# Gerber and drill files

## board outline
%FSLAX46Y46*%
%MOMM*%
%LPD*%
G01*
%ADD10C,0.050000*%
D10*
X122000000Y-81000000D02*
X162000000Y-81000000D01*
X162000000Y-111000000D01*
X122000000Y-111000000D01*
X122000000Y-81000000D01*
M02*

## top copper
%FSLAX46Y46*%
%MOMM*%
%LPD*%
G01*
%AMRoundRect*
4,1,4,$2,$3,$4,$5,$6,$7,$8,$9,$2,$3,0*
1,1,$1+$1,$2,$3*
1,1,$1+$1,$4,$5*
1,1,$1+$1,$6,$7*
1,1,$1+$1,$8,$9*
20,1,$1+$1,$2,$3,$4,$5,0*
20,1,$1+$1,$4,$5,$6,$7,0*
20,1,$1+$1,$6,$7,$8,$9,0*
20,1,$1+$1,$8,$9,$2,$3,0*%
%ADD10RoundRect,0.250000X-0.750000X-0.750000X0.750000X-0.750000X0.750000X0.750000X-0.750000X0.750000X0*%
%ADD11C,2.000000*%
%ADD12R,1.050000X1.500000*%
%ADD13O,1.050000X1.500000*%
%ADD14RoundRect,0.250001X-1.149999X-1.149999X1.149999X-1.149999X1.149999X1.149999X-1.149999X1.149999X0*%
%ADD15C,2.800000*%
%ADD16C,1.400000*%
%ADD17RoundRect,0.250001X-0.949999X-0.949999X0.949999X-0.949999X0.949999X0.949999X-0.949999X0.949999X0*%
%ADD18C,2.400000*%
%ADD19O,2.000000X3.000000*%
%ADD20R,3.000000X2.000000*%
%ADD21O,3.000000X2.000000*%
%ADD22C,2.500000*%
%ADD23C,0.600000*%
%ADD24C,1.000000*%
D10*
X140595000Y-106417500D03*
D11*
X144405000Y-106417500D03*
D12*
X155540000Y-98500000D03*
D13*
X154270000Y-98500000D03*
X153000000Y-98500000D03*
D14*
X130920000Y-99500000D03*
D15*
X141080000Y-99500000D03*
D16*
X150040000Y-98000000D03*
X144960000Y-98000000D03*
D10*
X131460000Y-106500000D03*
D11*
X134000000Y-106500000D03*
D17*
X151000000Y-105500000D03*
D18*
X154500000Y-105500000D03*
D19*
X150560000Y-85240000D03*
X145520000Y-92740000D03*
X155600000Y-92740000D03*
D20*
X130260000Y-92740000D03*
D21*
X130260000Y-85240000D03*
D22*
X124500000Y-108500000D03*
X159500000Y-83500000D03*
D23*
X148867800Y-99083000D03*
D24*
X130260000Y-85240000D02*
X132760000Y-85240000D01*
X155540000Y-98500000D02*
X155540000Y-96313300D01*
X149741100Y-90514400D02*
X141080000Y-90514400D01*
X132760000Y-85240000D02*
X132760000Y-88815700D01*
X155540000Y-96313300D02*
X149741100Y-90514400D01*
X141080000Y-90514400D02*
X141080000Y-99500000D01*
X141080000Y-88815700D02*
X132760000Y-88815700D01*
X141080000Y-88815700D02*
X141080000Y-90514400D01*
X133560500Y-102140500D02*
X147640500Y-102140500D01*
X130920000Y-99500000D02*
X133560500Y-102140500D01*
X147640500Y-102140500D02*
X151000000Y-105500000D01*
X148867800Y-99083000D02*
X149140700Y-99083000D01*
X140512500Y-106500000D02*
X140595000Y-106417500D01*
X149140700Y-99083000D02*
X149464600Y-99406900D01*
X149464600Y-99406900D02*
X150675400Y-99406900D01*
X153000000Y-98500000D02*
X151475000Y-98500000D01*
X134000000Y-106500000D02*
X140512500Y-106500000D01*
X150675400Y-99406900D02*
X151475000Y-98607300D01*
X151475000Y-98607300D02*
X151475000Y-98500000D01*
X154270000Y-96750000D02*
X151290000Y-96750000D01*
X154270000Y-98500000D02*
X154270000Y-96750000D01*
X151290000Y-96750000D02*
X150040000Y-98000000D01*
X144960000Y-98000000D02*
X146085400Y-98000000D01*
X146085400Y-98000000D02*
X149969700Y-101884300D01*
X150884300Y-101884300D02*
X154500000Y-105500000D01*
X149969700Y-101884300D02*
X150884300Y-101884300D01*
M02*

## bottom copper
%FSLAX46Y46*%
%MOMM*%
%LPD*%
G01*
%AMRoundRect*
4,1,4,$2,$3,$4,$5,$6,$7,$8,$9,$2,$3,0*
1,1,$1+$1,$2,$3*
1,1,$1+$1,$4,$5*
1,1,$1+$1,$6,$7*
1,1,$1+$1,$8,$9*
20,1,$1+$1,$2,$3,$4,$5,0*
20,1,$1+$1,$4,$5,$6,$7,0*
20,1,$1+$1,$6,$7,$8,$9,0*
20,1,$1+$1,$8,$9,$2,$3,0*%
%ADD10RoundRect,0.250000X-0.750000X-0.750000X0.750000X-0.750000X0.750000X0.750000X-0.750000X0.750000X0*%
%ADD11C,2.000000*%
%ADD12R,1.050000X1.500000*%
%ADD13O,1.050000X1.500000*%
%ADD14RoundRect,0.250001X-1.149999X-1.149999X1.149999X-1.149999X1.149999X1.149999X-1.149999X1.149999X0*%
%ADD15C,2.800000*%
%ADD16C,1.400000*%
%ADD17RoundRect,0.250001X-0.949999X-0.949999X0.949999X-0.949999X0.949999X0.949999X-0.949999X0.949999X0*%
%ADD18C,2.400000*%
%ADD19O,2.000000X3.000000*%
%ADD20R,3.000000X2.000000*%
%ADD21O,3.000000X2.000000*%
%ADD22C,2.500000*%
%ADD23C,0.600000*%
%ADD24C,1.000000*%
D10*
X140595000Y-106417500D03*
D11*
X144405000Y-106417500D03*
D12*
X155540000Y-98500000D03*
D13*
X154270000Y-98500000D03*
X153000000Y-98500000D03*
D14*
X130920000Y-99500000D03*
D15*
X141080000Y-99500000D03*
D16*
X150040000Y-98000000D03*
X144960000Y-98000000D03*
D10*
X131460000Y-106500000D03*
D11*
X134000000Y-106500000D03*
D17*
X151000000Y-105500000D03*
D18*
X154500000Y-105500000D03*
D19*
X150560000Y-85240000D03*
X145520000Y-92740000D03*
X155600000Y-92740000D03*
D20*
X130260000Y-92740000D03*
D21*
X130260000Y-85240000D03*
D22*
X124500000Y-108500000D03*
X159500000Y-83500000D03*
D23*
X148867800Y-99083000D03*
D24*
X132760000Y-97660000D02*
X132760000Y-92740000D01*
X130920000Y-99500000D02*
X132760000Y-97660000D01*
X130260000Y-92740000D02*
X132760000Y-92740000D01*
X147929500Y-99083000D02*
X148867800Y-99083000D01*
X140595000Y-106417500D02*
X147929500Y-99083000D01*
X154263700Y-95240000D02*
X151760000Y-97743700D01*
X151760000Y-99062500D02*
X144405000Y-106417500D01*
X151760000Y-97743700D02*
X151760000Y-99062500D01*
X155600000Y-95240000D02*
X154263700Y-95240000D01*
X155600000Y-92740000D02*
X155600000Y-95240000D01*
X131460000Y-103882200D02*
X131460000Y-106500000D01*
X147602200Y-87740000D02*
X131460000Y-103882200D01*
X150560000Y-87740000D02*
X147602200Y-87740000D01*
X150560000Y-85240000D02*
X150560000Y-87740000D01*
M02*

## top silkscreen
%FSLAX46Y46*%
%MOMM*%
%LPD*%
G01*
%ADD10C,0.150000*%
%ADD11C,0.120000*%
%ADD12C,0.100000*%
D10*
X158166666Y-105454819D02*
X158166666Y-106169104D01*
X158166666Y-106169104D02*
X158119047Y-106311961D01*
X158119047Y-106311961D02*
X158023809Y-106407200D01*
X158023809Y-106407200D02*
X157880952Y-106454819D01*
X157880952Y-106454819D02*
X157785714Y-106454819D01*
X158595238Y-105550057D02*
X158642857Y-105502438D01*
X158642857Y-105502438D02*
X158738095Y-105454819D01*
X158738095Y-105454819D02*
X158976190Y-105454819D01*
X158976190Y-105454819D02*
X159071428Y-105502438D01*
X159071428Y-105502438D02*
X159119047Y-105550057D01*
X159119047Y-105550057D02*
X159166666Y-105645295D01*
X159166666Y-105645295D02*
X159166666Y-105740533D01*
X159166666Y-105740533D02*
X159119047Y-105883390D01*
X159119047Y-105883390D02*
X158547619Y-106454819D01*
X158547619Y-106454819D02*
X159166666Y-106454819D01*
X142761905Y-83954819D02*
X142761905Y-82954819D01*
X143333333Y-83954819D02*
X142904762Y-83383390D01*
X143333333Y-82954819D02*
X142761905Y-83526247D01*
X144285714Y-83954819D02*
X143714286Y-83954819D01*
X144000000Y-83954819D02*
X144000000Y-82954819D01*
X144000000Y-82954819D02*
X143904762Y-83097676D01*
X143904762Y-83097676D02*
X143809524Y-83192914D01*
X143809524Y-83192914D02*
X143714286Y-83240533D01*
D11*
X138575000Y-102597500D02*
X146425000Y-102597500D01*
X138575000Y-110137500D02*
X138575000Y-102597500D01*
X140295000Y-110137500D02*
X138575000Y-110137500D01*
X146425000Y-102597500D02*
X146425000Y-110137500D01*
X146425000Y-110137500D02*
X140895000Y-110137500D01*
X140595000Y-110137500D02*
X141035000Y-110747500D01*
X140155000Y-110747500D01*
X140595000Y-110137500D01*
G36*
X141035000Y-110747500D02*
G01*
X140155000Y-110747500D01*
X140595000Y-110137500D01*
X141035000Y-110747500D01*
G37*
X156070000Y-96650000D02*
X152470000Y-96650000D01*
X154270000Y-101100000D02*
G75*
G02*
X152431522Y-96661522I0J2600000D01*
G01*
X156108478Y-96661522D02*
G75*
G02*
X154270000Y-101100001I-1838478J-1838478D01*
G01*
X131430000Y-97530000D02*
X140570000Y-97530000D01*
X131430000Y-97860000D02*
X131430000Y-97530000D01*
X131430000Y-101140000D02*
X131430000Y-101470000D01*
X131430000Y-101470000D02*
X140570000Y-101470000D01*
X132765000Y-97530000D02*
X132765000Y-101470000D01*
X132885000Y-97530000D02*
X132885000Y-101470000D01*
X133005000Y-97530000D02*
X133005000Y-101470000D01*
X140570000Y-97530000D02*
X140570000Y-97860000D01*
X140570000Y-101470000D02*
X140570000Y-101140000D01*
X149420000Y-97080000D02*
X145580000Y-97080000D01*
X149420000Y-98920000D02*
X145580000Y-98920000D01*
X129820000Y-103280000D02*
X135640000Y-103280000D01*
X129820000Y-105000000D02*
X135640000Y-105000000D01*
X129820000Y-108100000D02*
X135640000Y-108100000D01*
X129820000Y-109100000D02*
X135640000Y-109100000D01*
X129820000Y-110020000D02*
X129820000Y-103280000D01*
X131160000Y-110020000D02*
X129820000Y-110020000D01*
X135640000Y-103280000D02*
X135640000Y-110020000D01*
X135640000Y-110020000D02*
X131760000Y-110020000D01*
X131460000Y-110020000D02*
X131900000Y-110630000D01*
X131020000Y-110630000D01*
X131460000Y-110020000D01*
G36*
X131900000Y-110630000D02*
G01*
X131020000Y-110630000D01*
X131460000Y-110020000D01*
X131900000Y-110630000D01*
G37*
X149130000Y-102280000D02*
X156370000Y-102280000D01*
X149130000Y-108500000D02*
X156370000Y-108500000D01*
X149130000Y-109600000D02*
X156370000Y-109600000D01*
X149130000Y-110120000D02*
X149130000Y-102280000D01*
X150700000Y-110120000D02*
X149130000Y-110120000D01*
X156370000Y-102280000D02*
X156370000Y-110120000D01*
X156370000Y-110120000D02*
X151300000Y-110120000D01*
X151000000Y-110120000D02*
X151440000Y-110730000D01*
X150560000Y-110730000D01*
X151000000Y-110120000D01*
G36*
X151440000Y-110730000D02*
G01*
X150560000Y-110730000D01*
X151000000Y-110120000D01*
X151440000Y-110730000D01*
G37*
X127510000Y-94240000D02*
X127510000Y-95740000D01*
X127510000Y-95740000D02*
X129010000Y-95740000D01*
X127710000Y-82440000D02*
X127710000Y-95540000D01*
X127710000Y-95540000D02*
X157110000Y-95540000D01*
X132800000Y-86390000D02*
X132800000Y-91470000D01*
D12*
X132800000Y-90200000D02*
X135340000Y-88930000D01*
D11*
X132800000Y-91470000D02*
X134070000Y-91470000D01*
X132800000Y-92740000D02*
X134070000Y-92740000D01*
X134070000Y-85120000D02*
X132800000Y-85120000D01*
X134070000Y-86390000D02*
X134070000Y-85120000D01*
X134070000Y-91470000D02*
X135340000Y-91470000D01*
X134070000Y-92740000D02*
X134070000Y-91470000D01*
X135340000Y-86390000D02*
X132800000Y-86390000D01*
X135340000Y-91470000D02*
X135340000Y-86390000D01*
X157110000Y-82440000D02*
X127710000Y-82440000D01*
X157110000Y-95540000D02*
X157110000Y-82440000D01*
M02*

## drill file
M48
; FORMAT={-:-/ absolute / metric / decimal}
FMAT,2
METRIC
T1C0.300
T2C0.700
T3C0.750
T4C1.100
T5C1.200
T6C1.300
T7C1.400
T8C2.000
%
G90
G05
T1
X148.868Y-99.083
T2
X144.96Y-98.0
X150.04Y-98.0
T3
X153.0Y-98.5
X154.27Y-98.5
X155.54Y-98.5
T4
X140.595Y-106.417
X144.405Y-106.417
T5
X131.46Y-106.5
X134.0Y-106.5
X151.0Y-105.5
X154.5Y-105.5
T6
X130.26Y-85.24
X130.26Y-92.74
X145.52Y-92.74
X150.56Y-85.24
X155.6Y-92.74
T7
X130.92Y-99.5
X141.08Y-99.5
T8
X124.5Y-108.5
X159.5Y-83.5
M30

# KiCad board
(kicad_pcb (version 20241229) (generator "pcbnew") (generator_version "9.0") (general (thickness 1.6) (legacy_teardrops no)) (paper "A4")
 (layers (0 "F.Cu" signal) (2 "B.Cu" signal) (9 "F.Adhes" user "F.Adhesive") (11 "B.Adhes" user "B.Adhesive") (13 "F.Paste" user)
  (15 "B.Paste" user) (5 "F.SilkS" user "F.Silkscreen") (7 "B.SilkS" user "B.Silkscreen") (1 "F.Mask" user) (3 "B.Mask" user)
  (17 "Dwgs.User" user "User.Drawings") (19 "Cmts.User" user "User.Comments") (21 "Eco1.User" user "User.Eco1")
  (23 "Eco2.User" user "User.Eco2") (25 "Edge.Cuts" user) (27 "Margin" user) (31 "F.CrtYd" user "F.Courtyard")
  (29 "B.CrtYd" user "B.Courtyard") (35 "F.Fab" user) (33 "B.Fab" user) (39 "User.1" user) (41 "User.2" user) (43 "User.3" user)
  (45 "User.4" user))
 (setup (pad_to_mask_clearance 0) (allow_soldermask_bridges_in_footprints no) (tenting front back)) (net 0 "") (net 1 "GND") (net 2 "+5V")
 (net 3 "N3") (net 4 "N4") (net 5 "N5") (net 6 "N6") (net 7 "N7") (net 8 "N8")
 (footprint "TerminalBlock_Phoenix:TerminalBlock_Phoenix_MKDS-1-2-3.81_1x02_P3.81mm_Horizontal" (layer "F.Cu") (at 140.595 106.4175)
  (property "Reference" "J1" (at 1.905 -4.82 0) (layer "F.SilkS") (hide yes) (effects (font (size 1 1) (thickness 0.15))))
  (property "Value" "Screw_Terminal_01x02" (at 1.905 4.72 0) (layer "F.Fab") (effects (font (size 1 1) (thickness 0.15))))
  (fp_line (start -2.02 -3.82) (end 5.83 -3.82) (stroke (width 0.12) (type solid)) (layer "F.SilkS"))
  (fp_line (start -2.02 3.72) (end -2.02 -3.82) (stroke (width 0.12) (type solid)) (layer "F.SilkS"))
  (fp_line (start -0.3 3.72) (end -2.02 3.72) (stroke (width 0.12) (type solid)) (layer "F.SilkS"))
  (fp_line (start 5.83 -3.82) (end 5.83 3.72) (stroke (width 0.12) (type solid)) (layer "F.SilkS"))
  (fp_line (start 5.83 3.72) (end 0.3 3.72) (stroke (width 0.12) (type solid)) (layer "F.SilkS"))
  (fp_poly (pts (xy 0 3.72) (xy 0.44 4.33) (xy -0.44 4.33)) (stroke (width 0.12) (type solid)) (fill yes) (layer "F.SilkS"))
  (pad "1" thru_hole roundrect (at 0 0) (size 2 2) (drill 1.1) (layers "*.Cu" "*.Mask") (remove_unused_layers no) (roundrect_rratio 0.125)
   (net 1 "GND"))
  (pad "2" thru_hole circle (at 3.81 0) (size 2 2) (drill 1.1) (layers "*.Cu" "*.Mask") (remove_unused_layers no) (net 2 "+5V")))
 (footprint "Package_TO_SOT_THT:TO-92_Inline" (layer "F.Cu") (at 155.54 98.5 180)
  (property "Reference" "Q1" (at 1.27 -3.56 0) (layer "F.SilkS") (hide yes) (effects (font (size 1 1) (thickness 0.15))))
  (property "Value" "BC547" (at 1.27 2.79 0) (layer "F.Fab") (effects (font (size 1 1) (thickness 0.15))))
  (fp_line (start -0.53 1.85) (end 3.07 1.85) (stroke (width 0.12) (type solid)) (layer "F.SilkS"))
  (fp_arc (start 1.27 -2.6) (mid 3.672087 -0.994977) (end 3.108478 1.838478) (stroke (width 0.12) (type solid)) (layer "F.SilkS"))
  (fp_arc (start -0.568478 1.838478) (mid -1.132087 -0.994977) (end 1.27 -2.6) (stroke (width 0.12) (type solid)) (layer "F.SilkS"))
  (pad "1" thru_hole rect (at 0 0 180) (size 1.05 1.5) (drill 0.75) (layers "*.Cu" "*.Mask") (remove_unused_layers no) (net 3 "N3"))
  (pad "2" thru_hole oval (at 1.27 0 180) (size 1.05 1.5) (drill 0.75) (layers "*.Cu" "*.Mask") (remove_unused_layers no) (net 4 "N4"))
  (pad "3" thru_hole oval (at 2.54 0 180) (size 1.05 1.5) (drill 0.75) (layers "*.Cu" "*.Mask") (remove_unused_layers no) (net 1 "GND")))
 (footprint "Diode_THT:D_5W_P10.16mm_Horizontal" (layer "F.Cu") (at 130.92 99.5)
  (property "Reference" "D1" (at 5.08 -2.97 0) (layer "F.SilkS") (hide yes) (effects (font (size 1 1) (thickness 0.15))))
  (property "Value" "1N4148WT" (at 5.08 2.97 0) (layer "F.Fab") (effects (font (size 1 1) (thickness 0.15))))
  (fp_line (start 0.51 -1.97) (end 9.65 -1.97) (stroke (width 0.12) (type solid)) (layer "F.SilkS"))
  (fp_line (start 0.51 -1.64) (end 0.51 -1.97) (stroke (width 0.12) (type solid)) (layer "F.SilkS"))
  (fp_line (start 0.51 1.64) (end 0.51 1.97) (stroke (width 0.12) (type solid)) (layer "F.SilkS"))
  (fp_line (start 0.51 1.97) (end 9.65 1.97) (stroke (width 0.12) (type solid)) (layer "F.SilkS"))
  (fp_line (start 1.845 -1.97) (end 1.845 1.97) (stroke (width 0.12) (type solid)) (layer "F.SilkS"))
  (fp_line (start 1.965 -1.97) (end 1.965 1.97) (stroke (width 0.12) (type solid)) (layer "F.SilkS"))
  (fp_line (start 2.085 -1.97) (end 2.085 1.97) (stroke (width 0.12) (type solid)) (layer "F.SilkS"))
  (fp_line (start 9.65 -1.97) (end 9.65 -1.64) (stroke (width 0.12) (type solid)) (layer "F.SilkS"))
  (fp_line (start 9.65 1.97) (end 9.65 1.64) (stroke (width 0.12) (type solid)) (layer "F.SilkS"))
  (pad "1" thru_hole roundrect (at 0 0) (size 2.8 2.8) (drill 1.4) (layers "*.Cu" "*.Mask") (remove_unused_layers no)
   (roundrect_rratio 0.089286) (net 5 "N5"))
  (pad "2" thru_hole circle (at 10.16 0) (size 2.8 2.8) (drill 1.4) (layers "*.Cu" "*.Mask") (remove_unused_layers no) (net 3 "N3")))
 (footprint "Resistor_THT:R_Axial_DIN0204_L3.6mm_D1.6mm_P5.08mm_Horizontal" (layer "F.Cu") (at 150.04 98 180)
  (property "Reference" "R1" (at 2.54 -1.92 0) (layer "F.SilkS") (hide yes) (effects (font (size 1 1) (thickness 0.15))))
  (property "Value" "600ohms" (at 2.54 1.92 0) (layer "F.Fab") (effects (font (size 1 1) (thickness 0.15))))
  (fp_line (start 0.62 0.92) (end 4.46 0.92) (stroke (width 0.12) (type solid)) (layer "F.SilkS"))
  (fp_line (start 0.62 -0.92) (end 4.46 -0.92) (stroke (width 0.12) (type solid)) (layer "F.SilkS"))
  (pad "1" thru_hole circle (at 0 0 180) (size 1.4 1.4) (drill 0.7) (layers "*.Cu" "*.Mask") (remove_unused_layers no) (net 4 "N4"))
  (pad "2" thru_hole circle (at 5.08 0 180) (size 1.4 1.4) (drill 0.7) (layers "*.Cu" "*.Mask") (remove_unused_layers no) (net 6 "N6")))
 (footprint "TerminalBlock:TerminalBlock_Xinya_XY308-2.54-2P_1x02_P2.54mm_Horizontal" (layer "F.Cu") (at 131.46 106.5)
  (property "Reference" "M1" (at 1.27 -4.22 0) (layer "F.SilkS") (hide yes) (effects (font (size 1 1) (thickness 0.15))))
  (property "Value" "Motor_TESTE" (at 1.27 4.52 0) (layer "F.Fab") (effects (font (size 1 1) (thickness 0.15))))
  (fp_line (start -1.64 -3.22) (end 4.18 -3.22) (stroke (width 0.12) (type solid)) (layer "F.SilkS"))
  (fp_line (start -1.64 -1.5) (end 4.18 -1.5) (stroke (width 0.12) (type solid)) (layer "F.SilkS"))
  (fp_line (start -1.64 1.6) (end 4.18 1.6) (stroke (width 0.12) (type solid)) (layer "F.SilkS"))
  (fp_line (start -1.64 2.6) (end 4.18 2.6) (stroke (width 0.12) (type solid)) (layer "F.SilkS"))
  (fp_line (start -1.64 3.52) (end -1.64 -3.22) (stroke (width 0.12) (type solid)) (layer "F.SilkS"))
  (fp_line (start -0.3 3.52) (end -1.64 3.52) (stroke (width 0.12) (type solid)) (layer "F.SilkS"))
  (fp_line (start 4.18 -3.22) (end 4.18 3.52) (stroke (width 0.12) (type solid)) (layer "F.SilkS"))
  (fp_line (start 4.18 3.52) (end 0.3 3.52) (stroke (width 0.12) (type solid)) (layer "F.SilkS"))
  (fp_poly (pts (xy 0 3.52) (xy 0.44 4.13) (xy -0.44 4.13)) (stroke (width 0.12) (type solid)) (fill yes) (layer "F.SilkS"))
  (pad "1" thru_hole roundrect (at 0 0) (size 2 2) (drill 1.2) (layers "*.Cu" "*.Mask") (remove_unused_layers no) (roundrect_rratio 0.125)
   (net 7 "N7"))
  (pad "2" thru_hole circle (at 2.54 0) (size 2 2) (drill 1.2) (layers "*.Cu" "*.Mask") (remove_unused_layers no) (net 1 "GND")))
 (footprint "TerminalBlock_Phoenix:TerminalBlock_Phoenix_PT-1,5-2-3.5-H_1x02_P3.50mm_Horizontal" (layer "F.Cu") (at 151 105.5)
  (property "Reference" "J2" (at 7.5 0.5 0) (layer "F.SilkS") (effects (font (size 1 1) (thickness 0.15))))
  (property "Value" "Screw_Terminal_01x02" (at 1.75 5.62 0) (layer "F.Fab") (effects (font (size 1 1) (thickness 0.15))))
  (fp_line (start -1.87 -3.22) (end 5.37 -3.22) (stroke (width 0.12) (type solid)) (layer "F.SilkS"))
  (fp_line (start -1.87 3) (end 5.37 3) (stroke (width 0.12) (type solid)) (layer "F.SilkS"))
  (fp_line (start -1.87 4.1) (end 5.37 4.1) (stroke (width 0.12) (type solid)) (layer "F.SilkS"))
  (fp_line (start -1.87 4.62) (end -1.87 -3.22) (stroke (width 0.12) (type solid)) (layer "F.SilkS"))
  (fp_line (start -0.3 4.62) (end -1.87 4.62) (stroke (width 0.12) (type solid)) (layer "F.SilkS"))
  (fp_line (start 5.37 -3.22) (end 5.37 4.62) (stroke (width 0.12) (type solid)) (layer "F.SilkS"))
  (fp_line (start 5.37 4.62) (end 0.3 4.62) (stroke (width 0.12) (type solid)) (layer "F.SilkS"))
  (fp_poly (pts (xy 0 4.62) (xy 0.44 5.23) (xy -0.44 5.23)) (stroke (width 0.12) (type solid)) (fill yes) (layer "F.SilkS"))
  (pad "1" thru_hole roundrect (at 0 0) (size 2.4 2.4) (drill 1.2) (layers "*.Cu" "*.Mask") (remove_unused_layers no)
   (roundrect_rratio 0.104167) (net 5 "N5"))
  (pad "2" thru_hole circle (at 3.5 0) (size 2.4 2.4) (drill 1.2) (layers "*.Cu" "*.Mask") (remove_unused_layers no) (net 6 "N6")))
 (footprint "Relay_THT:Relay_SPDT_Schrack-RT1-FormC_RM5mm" (layer "F.Cu") (at 130.26 92.74)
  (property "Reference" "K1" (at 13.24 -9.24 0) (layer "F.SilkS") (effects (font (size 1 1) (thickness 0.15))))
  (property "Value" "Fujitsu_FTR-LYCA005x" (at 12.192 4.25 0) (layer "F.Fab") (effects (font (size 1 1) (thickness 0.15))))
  (fp_line (start -2.75 1.5) (end -2.75 3) (stroke (width 0.12) (type solid)) (layer "F.SilkS"))
  (fp_line (start -2.75 3) (end -1.25 3) (stroke (width 0.12) (type solid)) (layer "F.SilkS"))
  (fp_line (start -2.55 -10.3) (end -2.55 2.8) (stroke (width 0.12) (type solid)) (layer "F.SilkS"))
  (fp_line (start -2.55 2.8) (end 26.85 2.8) (stroke (width 0.12) (type solid)) (layer "F.SilkS"))
  (fp_line (start 2.54 -6.35) (end 2.54 -1.27) (stroke (width 0.12) (type solid)) (layer "F.SilkS"))
  (fp_line (start 2.54 -2.54) (end 5.08 -3.81) (stroke (width 0.1) (type solid)) (layer "F.SilkS"))
  (fp_line (start 2.54 -1.27) (end 3.81 -1.27) (stroke (width 0.12) (type solid)) (layer "F.SilkS"))
  (fp_line (start 2.54 0) (end 3.81 0) (stroke (width 0.12) (type solid)) (layer "F.SilkS"))
  (fp_line (start 3.81 -7.62) (end 2.54 -7.62) (stroke (width 0.12) (type solid)) (layer "F.SilkS"))
  (fp_line (start 3.81 -6.35) (end 3.81 -7.62) (stroke (width 0.12) (type solid)) (layer "F.SilkS"))
  (fp_line (start 3.81 -1.27) (end 5.08 -1.27) (stroke (width 0.12) (type solid)) (layer "F.SilkS"))
  (fp_line (start 3.81 0) (end 3.81 -1.27) (stroke (width 0.12) (type solid)) (layer "F.SilkS"))
  (fp_line (start 5.08 -6.35) (end 2.54 -6.35) (stroke (width 0.12) (type solid)) (layer "F.SilkS"))
  (fp_line (start 5.08 -1.27) (end 5.08 -6.35) (stroke (width 0.12) (type solid)) (layer "F.SilkS"))
  (fp_line (start 26.85 -10.3) (end -2.55 -10.3) (stroke (width 0.12) (type solid)) (layer "F.SilkS"))
  (fp_line (start 26.85 2.8) (end 26.85 -10.3) (stroke (width 0.12) (type solid)) (layer "F.SilkS"))
  (pad "11" thru_hole oval (at 20.3 -7.5 180) (size 2 3) (drill 1.3) (layers "*.Cu" "*.Mask") (remove_unused_layers no) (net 7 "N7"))
  (pad "12" thru_hole oval (at 15.26 0 180) (size 2 3) (drill 1.3) (layers "*.Cu" "*.Mask") (remove_unused_layers no) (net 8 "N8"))
  (pad "14" thru_hole oval (at 25.34 0 180) (size 2 3) (drill 1.3) (layers "*.Cu" "*.Mask") (remove_unused_layers no) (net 2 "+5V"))
  (pad "A1" thru_hole rect (at 0 0 180) (size 3 2) (drill 1.3) (layers "*.Cu" "*.Mask") (remove_unused_layers no) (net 5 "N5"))
  (pad "A2" thru_hole oval (at 0 -7.5 180) (size 3 2) (drill 1.3) (layers "*.Cu" "*.Mask") (remove_unused_layers no) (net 3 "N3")))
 (gr_rect (start 122 81) (end 162 111) (stroke (width 0.05) (type default)) (fill no) (layer "Edge.Cuts"))
 (via (at 124.5 108.5) (size 2.5) (drill 2) (layers "F.Cu" "B.Cu") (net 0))
 (via (at 159.5 83.5) (size 2.5) (drill 2) (layers "F.Cu" "B.Cu") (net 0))
 (segment (start 130.26 85.24) (end 132.76 85.24) (width 1) (layer "F.Cu") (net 3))
 (segment (start 155.54 98.5) (end 155.54 96.3133) (width 1) (layer "F.Cu") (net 3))
 (segment (start 149.7411 90.5144) (end 141.08 90.5144) (width 1) (layer "F.Cu") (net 3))
 (segment (start 132.76 85.24) (end 132.76 88.8157) (width 1) (layer "F.Cu") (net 3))
 (segment (start 155.54 96.3133) (end 149.7411 90.5144) (width 1) (layer "F.Cu") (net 3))
 (segment (start 141.08 90.5144) (end 141.08 99.5) (width 1) (layer "F.Cu") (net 3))
 (segment (start 141.08 88.8157) (end 132.76 88.8157) (width 1) (layer "F.Cu") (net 3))
 (segment (start 141.08 88.8157) (end 141.08 90.5144) (width 1) (layer "F.Cu") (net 3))
 (segment (start 133.5605 102.1405) (end 147.6405 102.1405) (width 1) (layer "F.Cu") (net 5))
 (segment (start 130.92 99.5) (end 133.5605 102.1405) (width 1) (layer "F.Cu") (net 5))
 (segment (start 147.6405 102.1405) (end 151 105.5) (width 1) (layer "F.Cu") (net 5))
 (segment (start 132.76 97.66) (end 132.76 92.74) (width 1) (layer "B.Cu") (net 5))
 (segment (start 130.92 99.5) (end 132.76 97.66) (width 1) (layer "B.Cu") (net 5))
 (segment (start 130.26 92.74) (end 132.76 92.74) (width 1) (layer "B.Cu") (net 5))
 (segment (start 148.8678 99.083) (end 149.1407 99.083) (width 1) (layer "F.Cu") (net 1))
 (segment (start 140.5125 106.5) (end 140.595 106.4175) (width 1) (layer "F.Cu") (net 1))
 (segment (start 149.1407 99.083) (end 149.4646 99.4069) (width 1) (layer "F.Cu") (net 1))
 (segment (start 149.4646 99.4069) (end 150.6754 99.4069) (width 1) (layer "F.Cu") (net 1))
 (segment (start 153 98.5) (end 151.475 98.5) (width 1) (layer "F.Cu") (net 1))
 (segment (start 134 106.5) (end 140.5125 106.5) (width 1) (layer "F.Cu") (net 1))
 (segment (start 150.6754 99.4069) (end 151.475 98.6073) (width 1) (layer "F.Cu") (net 1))
 (segment (start 151.475 98.6073) (end 151.475 98.5) (width 1) (layer "F.Cu") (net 1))
 (via (at 148.8678 99.083) (size 0.6) (drill 0.3) (layers "F.Cu" "B.Cu") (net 1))
 (segment (start 147.9295 99.083) (end 148.8678 99.083) (width 1) (layer "B.Cu") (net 1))
 (segment (start 140.595 106.4175) (end 147.9295 99.083) (width 1) (layer "B.Cu") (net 1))
 (segment (start 154.2637 95.24) (end 151.76 97.7437) (width 1) (layer "B.Cu") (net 2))
 (segment (start 151.76 99.0625) (end 144.405 106.4175) (width 1) (layer "B.Cu") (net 2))
 (segment (start 151.76 97.7437) (end 151.76 99.0625) (width 1) (layer "B.Cu") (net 2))
 (segment (start 155.6 95.24) (end 154.2637 95.24) (width 1) (layer "B.Cu") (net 2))
 (segment (start 155.6 92.74) (end 155.6 95.24) (width 1) (layer "B.Cu") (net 2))
 (segment (start 131.46 103.8822) (end 131.46 106.5) (width 1) (layer "B.Cu") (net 7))
 (segment (start 147.6022 87.74) (end 131.46 103.8822) (width 1) (layer "B.Cu") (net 7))
 (segment (start 150.56 87.74) (end 147.6022 87.74) (width 1) (layer "B.Cu") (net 7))
 (segment (start 150.56 85.24) (end 150.56 87.74) (width 1) (layer "B.Cu") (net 7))
 (segment (start 154.27 96.75) (end 151.29 96.75) (width 1) (layer "F.Cu") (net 4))
 (segment (start 154.27 98.5) (end 154.27 96.75) (width 1) (layer "F.Cu") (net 4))
 (segment (start 151.29 96.75) (end 150.04 98) (width 1) (layer "F.Cu") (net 4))
 (segment (start 144.96 98) (end 146.0854 98) (width 1) (layer "F.Cu") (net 6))
 (segment (start 146.0854 98) (end 149.9697 101.8843) (width 1) (layer "F.Cu") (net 6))
 (segment (start 150.8843 101.8843) (end 154.5 105.5) (width 1) (layer "F.Cu") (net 6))
 (segment (start 149.9697 101.8843) (end 150.8843 101.8843) (width 1) (layer "F.Cu") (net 6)))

